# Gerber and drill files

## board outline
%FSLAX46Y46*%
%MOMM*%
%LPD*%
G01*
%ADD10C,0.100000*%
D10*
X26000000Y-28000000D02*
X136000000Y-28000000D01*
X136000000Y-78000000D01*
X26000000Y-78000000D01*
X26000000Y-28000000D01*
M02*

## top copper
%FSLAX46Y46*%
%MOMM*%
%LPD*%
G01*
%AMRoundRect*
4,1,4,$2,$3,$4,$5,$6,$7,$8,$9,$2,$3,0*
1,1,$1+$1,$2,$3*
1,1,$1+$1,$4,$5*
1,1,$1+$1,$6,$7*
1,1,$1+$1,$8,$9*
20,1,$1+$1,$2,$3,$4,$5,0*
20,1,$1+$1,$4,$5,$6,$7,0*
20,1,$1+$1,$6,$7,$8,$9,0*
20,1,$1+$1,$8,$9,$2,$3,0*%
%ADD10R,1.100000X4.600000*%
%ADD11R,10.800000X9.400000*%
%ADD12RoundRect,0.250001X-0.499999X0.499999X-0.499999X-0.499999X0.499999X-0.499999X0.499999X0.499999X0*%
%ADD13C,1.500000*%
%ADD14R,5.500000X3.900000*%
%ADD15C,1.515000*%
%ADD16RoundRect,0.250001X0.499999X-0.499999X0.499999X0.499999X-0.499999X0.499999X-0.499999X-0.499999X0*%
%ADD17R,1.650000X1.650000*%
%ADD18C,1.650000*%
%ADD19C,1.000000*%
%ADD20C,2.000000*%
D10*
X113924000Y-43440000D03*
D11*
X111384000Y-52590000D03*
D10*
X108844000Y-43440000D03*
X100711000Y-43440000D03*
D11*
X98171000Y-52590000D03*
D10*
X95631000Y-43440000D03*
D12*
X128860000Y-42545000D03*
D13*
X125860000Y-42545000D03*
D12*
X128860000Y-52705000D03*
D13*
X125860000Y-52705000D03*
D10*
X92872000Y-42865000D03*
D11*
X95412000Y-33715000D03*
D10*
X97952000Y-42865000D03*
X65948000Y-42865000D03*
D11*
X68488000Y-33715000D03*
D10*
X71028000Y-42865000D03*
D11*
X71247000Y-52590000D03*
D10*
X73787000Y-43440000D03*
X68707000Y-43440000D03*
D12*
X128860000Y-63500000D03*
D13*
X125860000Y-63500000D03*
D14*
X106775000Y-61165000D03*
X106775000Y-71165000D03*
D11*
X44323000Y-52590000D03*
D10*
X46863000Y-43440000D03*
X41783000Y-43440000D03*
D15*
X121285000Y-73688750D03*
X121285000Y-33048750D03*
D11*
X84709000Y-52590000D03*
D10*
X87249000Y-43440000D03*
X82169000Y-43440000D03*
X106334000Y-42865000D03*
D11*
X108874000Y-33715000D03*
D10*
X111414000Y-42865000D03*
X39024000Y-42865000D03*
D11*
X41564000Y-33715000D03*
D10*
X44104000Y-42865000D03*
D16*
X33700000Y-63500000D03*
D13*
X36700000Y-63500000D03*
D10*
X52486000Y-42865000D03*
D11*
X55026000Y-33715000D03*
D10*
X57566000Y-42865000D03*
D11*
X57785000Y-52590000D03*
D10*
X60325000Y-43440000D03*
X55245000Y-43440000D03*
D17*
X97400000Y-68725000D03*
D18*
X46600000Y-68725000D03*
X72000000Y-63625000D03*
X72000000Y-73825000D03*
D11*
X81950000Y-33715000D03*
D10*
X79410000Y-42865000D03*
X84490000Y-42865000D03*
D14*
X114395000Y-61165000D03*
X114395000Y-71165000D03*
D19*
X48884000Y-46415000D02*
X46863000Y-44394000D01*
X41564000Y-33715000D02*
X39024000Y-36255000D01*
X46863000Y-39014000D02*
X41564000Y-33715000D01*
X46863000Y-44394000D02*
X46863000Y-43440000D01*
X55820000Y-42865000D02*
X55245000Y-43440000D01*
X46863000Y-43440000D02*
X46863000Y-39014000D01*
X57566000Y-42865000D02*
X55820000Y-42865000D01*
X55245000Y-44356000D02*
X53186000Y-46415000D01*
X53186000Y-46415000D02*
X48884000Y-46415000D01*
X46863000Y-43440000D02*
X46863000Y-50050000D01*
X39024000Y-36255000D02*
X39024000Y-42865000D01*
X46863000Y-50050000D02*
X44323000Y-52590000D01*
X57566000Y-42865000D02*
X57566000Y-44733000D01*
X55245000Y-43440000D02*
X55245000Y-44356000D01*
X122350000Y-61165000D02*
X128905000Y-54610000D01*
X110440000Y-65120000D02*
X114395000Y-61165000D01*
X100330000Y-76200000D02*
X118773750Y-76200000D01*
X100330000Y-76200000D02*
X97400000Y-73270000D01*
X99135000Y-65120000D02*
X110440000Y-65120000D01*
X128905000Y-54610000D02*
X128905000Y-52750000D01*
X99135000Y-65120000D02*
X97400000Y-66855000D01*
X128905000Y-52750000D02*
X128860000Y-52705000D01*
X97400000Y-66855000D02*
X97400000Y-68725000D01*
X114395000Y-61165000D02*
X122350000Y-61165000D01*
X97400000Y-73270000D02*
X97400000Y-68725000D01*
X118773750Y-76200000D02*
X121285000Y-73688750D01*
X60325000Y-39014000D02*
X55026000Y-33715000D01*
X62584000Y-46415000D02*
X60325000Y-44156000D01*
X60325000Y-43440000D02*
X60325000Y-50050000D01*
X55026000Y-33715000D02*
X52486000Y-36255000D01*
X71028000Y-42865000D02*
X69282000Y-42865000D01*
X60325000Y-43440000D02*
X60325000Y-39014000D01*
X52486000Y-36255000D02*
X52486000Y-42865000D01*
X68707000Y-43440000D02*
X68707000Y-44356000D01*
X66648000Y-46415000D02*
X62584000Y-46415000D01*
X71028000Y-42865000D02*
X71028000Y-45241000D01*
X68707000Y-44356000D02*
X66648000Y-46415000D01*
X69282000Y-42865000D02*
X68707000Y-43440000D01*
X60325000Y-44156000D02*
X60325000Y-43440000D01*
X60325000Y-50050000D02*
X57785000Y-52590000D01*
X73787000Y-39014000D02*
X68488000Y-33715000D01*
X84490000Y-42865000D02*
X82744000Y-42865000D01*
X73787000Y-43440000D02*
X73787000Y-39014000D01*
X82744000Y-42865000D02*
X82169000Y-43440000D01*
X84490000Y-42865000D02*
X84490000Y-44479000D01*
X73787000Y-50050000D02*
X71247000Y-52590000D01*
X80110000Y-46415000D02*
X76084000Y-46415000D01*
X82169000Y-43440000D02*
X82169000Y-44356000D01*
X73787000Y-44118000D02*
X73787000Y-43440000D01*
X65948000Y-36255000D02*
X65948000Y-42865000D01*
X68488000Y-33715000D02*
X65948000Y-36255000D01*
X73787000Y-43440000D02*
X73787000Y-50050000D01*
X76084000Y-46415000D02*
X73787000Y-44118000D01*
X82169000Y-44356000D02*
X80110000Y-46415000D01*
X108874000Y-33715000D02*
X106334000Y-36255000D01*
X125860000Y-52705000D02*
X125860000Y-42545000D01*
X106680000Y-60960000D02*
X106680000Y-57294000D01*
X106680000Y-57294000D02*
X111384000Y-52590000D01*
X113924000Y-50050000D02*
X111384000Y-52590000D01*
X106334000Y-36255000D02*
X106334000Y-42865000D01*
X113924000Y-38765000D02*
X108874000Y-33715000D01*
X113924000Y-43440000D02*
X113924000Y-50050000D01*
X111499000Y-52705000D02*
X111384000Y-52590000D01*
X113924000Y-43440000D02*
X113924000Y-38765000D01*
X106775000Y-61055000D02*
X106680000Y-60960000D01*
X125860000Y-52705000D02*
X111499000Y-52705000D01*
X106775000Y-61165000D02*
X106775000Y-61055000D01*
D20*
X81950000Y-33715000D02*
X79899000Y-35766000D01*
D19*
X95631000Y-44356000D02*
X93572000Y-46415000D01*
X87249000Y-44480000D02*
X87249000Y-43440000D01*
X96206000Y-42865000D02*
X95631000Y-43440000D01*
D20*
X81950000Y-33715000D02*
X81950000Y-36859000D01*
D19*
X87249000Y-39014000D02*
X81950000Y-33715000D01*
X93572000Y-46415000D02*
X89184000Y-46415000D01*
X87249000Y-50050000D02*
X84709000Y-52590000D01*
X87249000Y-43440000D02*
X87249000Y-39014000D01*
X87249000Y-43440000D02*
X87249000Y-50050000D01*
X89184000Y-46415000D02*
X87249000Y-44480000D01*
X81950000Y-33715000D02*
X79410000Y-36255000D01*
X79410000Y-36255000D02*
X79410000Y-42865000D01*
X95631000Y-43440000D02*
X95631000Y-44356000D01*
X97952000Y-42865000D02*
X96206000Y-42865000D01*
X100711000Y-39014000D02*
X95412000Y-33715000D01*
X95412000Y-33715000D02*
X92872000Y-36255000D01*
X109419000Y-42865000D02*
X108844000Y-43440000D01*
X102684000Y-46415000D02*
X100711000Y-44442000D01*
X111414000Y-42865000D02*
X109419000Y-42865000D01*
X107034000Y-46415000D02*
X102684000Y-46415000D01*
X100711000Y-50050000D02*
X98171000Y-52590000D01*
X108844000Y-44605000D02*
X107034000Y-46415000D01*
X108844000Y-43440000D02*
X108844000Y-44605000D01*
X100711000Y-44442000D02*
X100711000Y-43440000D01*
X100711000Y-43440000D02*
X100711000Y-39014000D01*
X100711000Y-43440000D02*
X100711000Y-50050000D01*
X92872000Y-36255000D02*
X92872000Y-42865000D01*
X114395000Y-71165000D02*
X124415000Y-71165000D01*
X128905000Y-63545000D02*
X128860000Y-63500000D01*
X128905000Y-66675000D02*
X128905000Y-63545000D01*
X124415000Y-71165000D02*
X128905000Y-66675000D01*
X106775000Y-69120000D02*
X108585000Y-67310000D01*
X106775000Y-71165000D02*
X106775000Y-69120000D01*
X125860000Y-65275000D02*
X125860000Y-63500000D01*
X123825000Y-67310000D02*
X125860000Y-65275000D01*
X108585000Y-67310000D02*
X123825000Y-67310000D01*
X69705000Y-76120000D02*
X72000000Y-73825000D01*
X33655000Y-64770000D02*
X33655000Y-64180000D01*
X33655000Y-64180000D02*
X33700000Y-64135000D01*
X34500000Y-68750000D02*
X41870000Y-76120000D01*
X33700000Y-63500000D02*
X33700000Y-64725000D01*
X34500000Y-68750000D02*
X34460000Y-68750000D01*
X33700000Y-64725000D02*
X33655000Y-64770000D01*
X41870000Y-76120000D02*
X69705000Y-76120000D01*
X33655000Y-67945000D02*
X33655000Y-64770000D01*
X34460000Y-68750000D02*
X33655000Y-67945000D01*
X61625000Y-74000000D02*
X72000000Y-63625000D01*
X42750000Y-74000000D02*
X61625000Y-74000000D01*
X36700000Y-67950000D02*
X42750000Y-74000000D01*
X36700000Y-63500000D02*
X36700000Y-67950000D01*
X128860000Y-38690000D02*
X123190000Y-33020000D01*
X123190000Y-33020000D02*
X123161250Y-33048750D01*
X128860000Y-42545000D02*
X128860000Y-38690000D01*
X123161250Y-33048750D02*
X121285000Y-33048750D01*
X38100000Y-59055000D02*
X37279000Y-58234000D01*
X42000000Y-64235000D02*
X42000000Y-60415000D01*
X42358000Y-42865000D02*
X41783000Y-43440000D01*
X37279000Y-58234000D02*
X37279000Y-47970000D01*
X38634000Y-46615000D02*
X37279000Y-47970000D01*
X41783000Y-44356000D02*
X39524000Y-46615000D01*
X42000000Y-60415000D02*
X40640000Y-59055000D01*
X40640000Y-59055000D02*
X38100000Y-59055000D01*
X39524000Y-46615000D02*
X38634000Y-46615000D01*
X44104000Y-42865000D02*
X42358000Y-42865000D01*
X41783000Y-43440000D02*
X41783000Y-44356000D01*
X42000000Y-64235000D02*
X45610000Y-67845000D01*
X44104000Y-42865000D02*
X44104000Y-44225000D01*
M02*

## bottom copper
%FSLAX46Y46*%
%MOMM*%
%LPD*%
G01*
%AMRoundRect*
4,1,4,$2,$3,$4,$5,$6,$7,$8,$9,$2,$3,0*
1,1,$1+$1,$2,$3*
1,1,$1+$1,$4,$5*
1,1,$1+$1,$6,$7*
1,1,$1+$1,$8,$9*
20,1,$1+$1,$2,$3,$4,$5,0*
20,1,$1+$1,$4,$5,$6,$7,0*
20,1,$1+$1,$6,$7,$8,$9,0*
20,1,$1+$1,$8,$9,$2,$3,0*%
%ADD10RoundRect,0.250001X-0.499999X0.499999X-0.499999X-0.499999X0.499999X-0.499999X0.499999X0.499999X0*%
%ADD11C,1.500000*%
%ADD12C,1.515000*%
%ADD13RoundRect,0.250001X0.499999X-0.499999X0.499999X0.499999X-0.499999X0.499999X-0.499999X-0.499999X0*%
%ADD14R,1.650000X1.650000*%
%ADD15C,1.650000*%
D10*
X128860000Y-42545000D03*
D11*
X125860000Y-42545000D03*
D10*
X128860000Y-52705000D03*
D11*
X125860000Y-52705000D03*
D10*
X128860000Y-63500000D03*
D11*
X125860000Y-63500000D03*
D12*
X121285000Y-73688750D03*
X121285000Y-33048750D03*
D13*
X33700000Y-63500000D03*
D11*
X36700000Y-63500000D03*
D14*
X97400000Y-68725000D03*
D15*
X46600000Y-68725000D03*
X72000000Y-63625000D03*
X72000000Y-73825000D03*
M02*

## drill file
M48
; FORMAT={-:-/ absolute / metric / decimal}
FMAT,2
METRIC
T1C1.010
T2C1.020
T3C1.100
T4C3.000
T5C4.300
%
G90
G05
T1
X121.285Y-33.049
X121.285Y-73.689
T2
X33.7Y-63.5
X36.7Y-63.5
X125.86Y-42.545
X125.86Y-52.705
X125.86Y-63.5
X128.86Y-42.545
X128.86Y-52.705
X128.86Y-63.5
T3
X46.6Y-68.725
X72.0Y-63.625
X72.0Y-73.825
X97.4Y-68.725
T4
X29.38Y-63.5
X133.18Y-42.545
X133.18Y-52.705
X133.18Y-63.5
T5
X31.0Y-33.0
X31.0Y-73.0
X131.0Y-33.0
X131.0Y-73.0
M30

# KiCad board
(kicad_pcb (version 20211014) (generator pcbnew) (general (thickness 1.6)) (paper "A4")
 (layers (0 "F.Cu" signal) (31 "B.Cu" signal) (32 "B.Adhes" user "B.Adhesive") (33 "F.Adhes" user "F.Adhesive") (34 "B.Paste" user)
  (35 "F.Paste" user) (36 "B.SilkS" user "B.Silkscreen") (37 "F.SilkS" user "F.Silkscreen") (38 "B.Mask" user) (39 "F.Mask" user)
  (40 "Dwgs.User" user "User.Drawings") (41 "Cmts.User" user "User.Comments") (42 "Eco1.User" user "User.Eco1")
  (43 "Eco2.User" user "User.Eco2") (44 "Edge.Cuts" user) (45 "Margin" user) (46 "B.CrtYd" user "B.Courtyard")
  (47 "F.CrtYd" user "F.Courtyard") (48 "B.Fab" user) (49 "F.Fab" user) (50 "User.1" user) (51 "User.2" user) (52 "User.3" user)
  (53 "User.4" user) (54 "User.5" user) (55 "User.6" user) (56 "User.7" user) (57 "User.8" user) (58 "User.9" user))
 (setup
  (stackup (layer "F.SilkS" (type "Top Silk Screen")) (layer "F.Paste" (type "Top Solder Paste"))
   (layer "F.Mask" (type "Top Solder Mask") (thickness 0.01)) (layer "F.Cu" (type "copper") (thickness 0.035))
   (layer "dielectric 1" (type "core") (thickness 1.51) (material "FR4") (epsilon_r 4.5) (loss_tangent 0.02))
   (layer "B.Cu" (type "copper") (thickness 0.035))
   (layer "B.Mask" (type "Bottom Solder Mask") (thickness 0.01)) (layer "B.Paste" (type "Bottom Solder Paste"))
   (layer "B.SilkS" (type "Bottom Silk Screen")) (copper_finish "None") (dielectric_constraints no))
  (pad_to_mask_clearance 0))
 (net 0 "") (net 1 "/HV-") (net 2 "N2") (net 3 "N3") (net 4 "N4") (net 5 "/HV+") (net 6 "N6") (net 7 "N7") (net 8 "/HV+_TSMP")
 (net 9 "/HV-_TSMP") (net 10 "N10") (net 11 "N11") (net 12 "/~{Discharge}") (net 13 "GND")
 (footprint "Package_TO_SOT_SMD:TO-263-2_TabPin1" (layer "F.Cu") (at 111.384 49.215 -90)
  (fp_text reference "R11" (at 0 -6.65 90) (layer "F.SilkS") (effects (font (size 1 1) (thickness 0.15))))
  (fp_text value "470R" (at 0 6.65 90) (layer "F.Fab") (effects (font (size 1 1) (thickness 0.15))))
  (pad "" smd rect (at 5.8 2.775 270) (size 4.55 5.25) (layers "F.Paste"))
  (pad "" smd rect (at 5.8 -2.775 270) (size 4.55 5.25) (layers "F.Paste"))
  (pad "" smd rect (at 0.95 -2.775 270) (size 4.55 5.25) (layers "F.Paste"))
  (pad "" smd rect (at 0.95 2.775 270) (size 4.55 5.25) (layers "F.Paste"))
  (pad "1" smd rect (at -5.775 -2.54 270) (size 4.6 1.1) (layers "F.Cu" "F.Paste" "F.Mask") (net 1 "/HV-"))
  (pad "1" smd rect (at 3.375 0 270) (size 9.4 10.8) (layers "F.Cu" "F.Mask") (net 1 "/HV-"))
  (pad "2" smd rect (at -5.775 2.54 270) (size 4.6 1.1) (layers "F.Cu" "F.Paste" "F.Mask") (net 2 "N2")))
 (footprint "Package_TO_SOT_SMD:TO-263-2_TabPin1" (layer "F.Cu") (at 98.171 49.215 -90)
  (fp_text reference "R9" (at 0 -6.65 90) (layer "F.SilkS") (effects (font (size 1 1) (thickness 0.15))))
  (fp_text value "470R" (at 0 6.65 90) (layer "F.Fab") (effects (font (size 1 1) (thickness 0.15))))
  (pad "" smd rect (at 0.95 -2.775 270) (size 4.55 5.25) (layers "F.Paste"))
  (pad "" smd rect (at 5.8 2.775 270) (size 4.55 5.25) (layers "F.Paste"))
  (pad "" smd rect (at 0.95 2.775 270) (size 4.55 5.25) (layers "F.Paste"))
  (pad "" smd rect (at 5.8 -2.775 270) (size 4.55 5.25) (layers "F.Paste"))
  (pad "1" smd rect (at -5.775 -2.54 270) (size 4.6 1.1) (layers "F.Cu" "F.Paste" "F.Mask") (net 2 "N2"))
  (pad "1" smd rect (at 3.375 0 270) (size 9.4 10.8) (layers "F.Cu" "F.Mask") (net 2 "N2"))
  (pad "2" smd rect (at -5.775 2.54 270) (size 4.6 1.1) (layers "F.Cu" "F.Paste" "F.Mask") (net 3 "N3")))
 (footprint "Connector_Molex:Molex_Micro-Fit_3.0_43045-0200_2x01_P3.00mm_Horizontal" (layer "F.Cu") (at 128.86 42.545 -90)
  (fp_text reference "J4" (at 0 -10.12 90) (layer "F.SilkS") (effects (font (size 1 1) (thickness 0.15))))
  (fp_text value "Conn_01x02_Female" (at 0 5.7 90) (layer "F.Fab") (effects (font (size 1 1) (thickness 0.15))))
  (pad "" np_thru_hole circle (at 0 -4.32 270) (size 3 3) (drill 3) (layers *.Cu *.Mask))
  (pad "1" thru_hole roundrect (at 0 0 270) (size 1.5 1.5) (drill 1.02) (layers *.Cu *.Mask) (roundrect_rratio 0.166667) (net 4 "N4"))
  (pad "2" thru_hole circle (at 0 3 270) (size 1.5 1.5) (drill 1.02) (layers *.Cu *.Mask) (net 1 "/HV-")))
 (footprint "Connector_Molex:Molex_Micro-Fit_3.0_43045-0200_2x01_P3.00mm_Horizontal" (layer "F.Cu") (at 128.86 52.705 -90)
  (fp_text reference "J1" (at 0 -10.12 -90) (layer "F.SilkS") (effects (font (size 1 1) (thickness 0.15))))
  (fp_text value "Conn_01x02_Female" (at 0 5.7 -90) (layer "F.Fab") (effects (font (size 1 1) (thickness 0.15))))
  (pad "" np_thru_hole circle (at 0 -4.32 270) (size 3 3) (drill 3) (layers *.Cu *.Mask))
  (pad "1" thru_hole roundrect (at 0 0 270) (size 1.5 1.5) (drill 1.02) (layers *.Cu *.Mask) (roundrect_rratio 0.1666673333) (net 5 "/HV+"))
  (pad "2" thru_hole circle (at 0 3 270) (size 1.5 1.5) (drill 1.02) (layers *.Cu *.Mask) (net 1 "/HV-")))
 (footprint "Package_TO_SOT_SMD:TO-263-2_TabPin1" (layer "F.Cu") (at 95.412 37.09 90)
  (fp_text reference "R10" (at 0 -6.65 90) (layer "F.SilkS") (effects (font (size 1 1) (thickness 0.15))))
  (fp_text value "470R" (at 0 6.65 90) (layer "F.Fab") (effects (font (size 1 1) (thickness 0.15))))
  (pad "" smd rect (at 5.8 -2.775 90) (size 4.55 5.25) (layers "F.Paste"))
  (pad "" smd rect (at 0.95 2.775 90) (size 4.55 5.25) (layers "F.Paste"))
  (pad "" smd rect (at 0.95 -2.775 90) (size 4.55 5.25) (layers "F.Paste"))
  (pad "" smd rect (at 5.8 2.775 90) (size 4.55 5.25) (layers "F.Paste"))
  (pad "1" smd rect (at -5.775 -2.54 90) (size 4.6 1.1) (layers "F.Cu" "F.Paste" "F.Mask") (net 2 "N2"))
  (pad "1" smd rect (at 3.375 0 90) (size 9.4 10.8) (layers "F.Cu" "F.Mask") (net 2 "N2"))
  (pad "2" smd rect (at -5.775 2.54 90) (size 4.6 1.1) (layers "F.Cu" "F.Paste" "F.Mask") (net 3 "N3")))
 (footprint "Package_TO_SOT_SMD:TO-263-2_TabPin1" (layer "F.Cu") (at 68.488 37.09 90)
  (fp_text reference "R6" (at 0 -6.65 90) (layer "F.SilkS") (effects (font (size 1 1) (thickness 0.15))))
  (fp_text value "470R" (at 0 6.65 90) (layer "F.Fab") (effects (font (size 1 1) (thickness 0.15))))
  (pad "" smd rect (at 0.95 2.775 90) (size 4.55 5.25) (layers "F.Paste"))
  (pad "" smd rect (at 5.8 -2.775 90) (size 4.55 5.25) (layers "F.Paste"))
  (pad "" smd rect (at 0.95 -2.775 90) (size 4.55 5.25) (layers "F.Paste"))
  (pad "" smd rect (at 5.8 2.775 90) (size 4.55 5.25) (layers "F.Paste"))
  (pad "1" smd rect (at -5.775 -2.54 90) (size 4.6 1.1) (layers "F.Cu" "F.Paste" "F.Mask") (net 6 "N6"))
  (pad "1" smd rect (at 3.375 0 90) (size 9.4 10.8) (layers "F.Cu" "F.Mask") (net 6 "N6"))
  (pad "2" smd rect (at -5.775 2.54 90) (size 4.6 1.1) (layers "F.Cu" "F.Paste" "F.Mask") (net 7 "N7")))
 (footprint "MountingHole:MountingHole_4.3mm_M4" (layer "F.Cu") (at 131 73)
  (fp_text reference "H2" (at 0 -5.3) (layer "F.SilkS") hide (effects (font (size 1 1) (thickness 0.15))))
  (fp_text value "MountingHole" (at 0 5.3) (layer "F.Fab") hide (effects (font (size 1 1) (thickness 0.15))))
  (pad "" np_thru_hole circle (at 0 0) (size 4.3 4.3) (drill 4.3) (layers *.Cu *.Mask)))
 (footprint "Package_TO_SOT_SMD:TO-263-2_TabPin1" (layer "F.Cu") (at 71.247 49.215 -90)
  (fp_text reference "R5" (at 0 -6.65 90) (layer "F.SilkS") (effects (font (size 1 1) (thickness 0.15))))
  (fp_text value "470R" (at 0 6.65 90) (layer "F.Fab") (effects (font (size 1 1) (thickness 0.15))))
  (pad "" smd rect (at 0.95 2.775 270) (size 4.55 5.25) (layers "F.Paste"))
  (pad "" smd rect (at 5.8 2.775 270) (size 4.55 5.25) (layers "F.Paste"))
  (pad "" smd rect (at 0.95 -2.775 270) (size 4.55 5.25) (layers "F.Paste"))
  (pad "" smd rect (at 5.8 -2.775 270) (size 4.55 5.25) (layers "F.Paste"))
  (pad "1" smd rect (at 3.375 0 270) (size 9.4 10.8) (layers "F.Cu" "F.Mask") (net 6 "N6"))
  (pad "1" smd rect (at -5.775 -2.54 270) (size 4.6 1.1) (layers "F.Cu" "F.Paste" "F.Mask") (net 6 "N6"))
  (pad "2" smd rect (at -5.775 2.54 270) (size 4.6 1.1) (layers "F.Cu" "F.Paste" "F.Mask") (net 7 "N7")))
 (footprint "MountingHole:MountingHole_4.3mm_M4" (layer "F.Cu") (at 31 73)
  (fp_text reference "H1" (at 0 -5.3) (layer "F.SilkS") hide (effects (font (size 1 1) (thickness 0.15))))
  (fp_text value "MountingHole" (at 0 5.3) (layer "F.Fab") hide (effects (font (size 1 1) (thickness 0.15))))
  (pad "" np_thru_hole circle (at 0 0) (size 4.3 4.3) (drill 4.3) (layers *.Cu *.Mask)))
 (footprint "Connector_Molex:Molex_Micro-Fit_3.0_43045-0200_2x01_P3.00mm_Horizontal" (layer "F.Cu") (at 128.86 63.5 -90)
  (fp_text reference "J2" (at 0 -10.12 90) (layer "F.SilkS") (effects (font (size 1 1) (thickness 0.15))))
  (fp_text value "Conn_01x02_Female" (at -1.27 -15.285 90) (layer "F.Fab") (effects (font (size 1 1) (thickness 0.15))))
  (pad "" np_thru_hole circle (at 0 -4.32 270) (size 3 3) (drill 3) (layers *.Cu *.Mask))
  (pad "1" thru_hole roundrect (at 0 0 270) (size 1.5 1.5) (drill 1.02) (layers *.Cu *.Mask) (roundrect_rratio 0.1666673333)
   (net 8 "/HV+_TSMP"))
  (pad "2" thru_hole circle (at 0 3 270) (size 1.5 1.5) (drill 1.02) (layers *.Cu *.Mask) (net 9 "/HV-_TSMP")))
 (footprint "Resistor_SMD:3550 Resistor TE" (layer "F.Cu") (at 104.025 59.215 -90)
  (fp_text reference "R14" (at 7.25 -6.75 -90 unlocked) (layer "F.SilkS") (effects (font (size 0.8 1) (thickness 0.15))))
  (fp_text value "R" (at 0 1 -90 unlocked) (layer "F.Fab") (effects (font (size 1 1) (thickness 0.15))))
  (pad "1" smd rect (at 1.95 -2.75 270) (size 3.9 5.5) (layers "F.Cu" "F.Paste" "F.Mask") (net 1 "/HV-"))
  (pad "2" smd rect (at 11.95 -2.75 270) (size 3.9 5.5) (layers "F.Cu" "F.Paste" "F.Mask") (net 9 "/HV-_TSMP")))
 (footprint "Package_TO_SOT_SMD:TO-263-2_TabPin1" (layer "F.Cu") (at 44.323 49.215 -90)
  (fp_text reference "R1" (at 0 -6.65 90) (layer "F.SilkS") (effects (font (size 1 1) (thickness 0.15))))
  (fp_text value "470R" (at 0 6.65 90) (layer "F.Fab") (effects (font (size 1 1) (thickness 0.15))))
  (pad "" smd rect (at 0.95 -2.775 270) (size 4.55 5.25) (layers "F.Paste"))
  (pad "" smd rect (at 5.8 2.775 270) (size 4.55 5.25) (layers "F.Paste"))
  (pad "" smd rect (at 5.8 -2.775 270) (size 4.55 5.25) (layers "F.Paste"))
  (pad "" smd rect (at 0.95 2.775 270) (size 4.55 5.25) (layers "F.Paste"))
  (pad "1" smd rect (at 3.375 0 270) (size 9.4 10.8) (layers "F.Cu" "F.Mask") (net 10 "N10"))
  (pad "1" smd rect (at -5.775 -2.54 270) (size 4.6 1.1) (layers "F.Cu" "F.Paste" "F.Mask") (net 10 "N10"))
  (pad "2" smd rect (at -5.775 2.54 270) (size 4.6 1.1) (layers "F.Cu" "F.Paste" "F.Mask") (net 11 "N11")))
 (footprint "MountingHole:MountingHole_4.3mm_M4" (layer "F.Cu") (at 131 33)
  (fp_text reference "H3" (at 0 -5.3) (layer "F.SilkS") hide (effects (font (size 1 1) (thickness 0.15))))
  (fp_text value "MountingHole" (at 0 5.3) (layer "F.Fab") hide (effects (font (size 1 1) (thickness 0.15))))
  (pad "" np_thru_hole circle (at 0 0) (size 4.3 4.3) (drill 4.3) (layers *.Cu *.Mask)))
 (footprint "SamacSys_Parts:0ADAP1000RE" (layer "F.Cu") (at 121.285 75.40875 90)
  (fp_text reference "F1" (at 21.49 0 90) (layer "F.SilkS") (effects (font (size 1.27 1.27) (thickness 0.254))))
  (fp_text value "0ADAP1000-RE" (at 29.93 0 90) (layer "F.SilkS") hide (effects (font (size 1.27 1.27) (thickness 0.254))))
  (pad "1" thru_hole circle (at 1.72 0 90) (size 1.515 1.515) (drill 1.01) (layers *.Cu *.Mask) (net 5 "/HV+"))
  (pad "2" thru_hole circle (at 42.36 0 90) (size 1.515 1.515) (drill 1.01) (layers *.Cu *.Mask) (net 4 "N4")))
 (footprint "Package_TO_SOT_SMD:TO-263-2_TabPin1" (layer "F.Cu") (at 84.709 49.215 -90)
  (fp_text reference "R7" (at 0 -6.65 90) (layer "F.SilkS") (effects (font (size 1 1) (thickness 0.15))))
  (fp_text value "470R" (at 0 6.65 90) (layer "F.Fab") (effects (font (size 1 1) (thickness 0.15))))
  (pad "" smd rect (at 0.95 2.775 270) (size 4.55 5.25) (layers "F.Paste"))
  (pad "" smd rect (at 0.95 -2.775 270) (size 4.55 5.25) (layers "F.Paste"))
  (pad "" smd rect (at 5.8 2.775 270) (size 4.55 5.25) (layers "F.Paste"))
  (pad "" smd rect (at 5.8 -2.775 270) (size 4.55 5.25) (layers "F.Paste"))
  (pad "1" smd rect (at 3.375 0 270) (size 9.4 10.8) (layers "F.Cu" "F.Mask") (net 3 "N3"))
  (pad "1" smd rect (at -5.775 -2.54 270) (size 4.6 1.1) (layers "F.Cu" "F.Paste" "F.Mask") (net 3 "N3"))
  (pad "2" smd rect (at -5.775 2.54 270) (size 4.6 1.1) (layers "F.Cu" "F.Paste" "F.Mask") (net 6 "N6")))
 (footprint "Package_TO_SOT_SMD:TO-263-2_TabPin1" (layer "F.Cu") (at 108.874 37.09 90)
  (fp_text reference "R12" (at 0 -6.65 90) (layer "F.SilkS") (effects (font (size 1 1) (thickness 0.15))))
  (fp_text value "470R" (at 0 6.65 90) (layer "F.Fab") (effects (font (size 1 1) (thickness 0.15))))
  (pad "" smd rect (at 5.8 2.775 90) (size 4.55 5.25) (layers "F.Paste"))
  (pad "" smd rect (at 0.95 -2.775 90) (size 4.55 5.25) (layers "F.Paste"))
  (pad "" smd rect (at 5.8 -2.775 90) (size 4.55 5.25) (layers "F.Paste"))
  (pad "" smd rect (at 0.95 2.775 90) (size 4.55 5.25) (layers "F.Paste"))
  (pad "1" smd rect (at -5.775 -2.54 90) (size 4.6 1.1) (layers "F.Cu" "F.Paste" "F.Mask") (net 1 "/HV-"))
  (pad "1" smd rect (at 3.375 0 90) (size 9.4 10.8) (layers "F.Cu" "F.Mask") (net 1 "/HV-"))
  (pad "2" smd rect (at -5.775 2.54 90) (size 4.6 1.1) (layers "F.Cu" "F.Paste" "F.Mask") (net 2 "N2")))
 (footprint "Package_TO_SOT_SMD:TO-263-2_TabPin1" (layer "F.Cu") (at 41.564 37.09 90)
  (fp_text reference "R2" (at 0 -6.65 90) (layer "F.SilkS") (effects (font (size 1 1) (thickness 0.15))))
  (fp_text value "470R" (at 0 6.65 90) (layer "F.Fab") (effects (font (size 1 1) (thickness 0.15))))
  (pad "" smd rect (at 5.8 2.775 90) (size 4.55 5.25) (layers "F.Paste"))
  (pad "" smd rect (at 5.8 -2.775 90) (size 4.55 5.25) (layers "F.Paste"))
  (pad "" smd rect (at 0.95 2.775 90) (size 4.55 5.25) (layers "F.Paste"))
  (pad "" smd rect (at 0.95 -2.775 90) (size 4.55 5.25) (layers "F.Paste"))
  (pad "1" smd rect (at -5.775 -2.54 90) (size 4.6 1.1) (layers "F.Cu" "F.Paste" "F.Mask") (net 10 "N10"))
  (pad "1" smd rect (at 3.375 0 90) (size 9.4 10.8) (layers "F.Cu" "F.Mask") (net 10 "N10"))
  (pad "2" smd rect (at -5.775 2.54 90) (size 4.6 1.1) (layers "F.Cu" "F.Paste" "F.Mask") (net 11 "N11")))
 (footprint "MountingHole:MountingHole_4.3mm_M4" (layer "F.Cu") (at 31 33)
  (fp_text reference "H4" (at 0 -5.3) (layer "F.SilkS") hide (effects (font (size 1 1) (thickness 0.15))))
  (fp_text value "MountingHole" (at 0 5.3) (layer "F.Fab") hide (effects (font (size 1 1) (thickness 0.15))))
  (pad "" np_thru_hole circle (at 0 0) (size 4.3 4.3) (drill 4.3) (layers *.Cu *.Mask)))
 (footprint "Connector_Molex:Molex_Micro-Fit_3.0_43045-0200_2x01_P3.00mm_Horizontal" (layer "F.Cu") (at 33.7 63.5 90)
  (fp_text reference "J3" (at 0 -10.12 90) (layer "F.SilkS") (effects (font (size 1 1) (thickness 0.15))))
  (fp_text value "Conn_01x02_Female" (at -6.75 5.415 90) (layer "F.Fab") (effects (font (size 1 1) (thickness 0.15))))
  (pad "" np_thru_hole circle (at 0 -4.32 90) (size 3 3) (drill 3) (layers *.Cu *.Mask))
  (pad "1" thru_hole roundrect (at 0 0 90) (size 1.5 1.5) (drill 1.02) (layers *.Cu *.Mask) (roundrect_rratio 0.1666673333)
   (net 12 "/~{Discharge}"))
  (pad "2" thru_hole circle (at 0 3 90) (size 1.5 1.5) (drill 1.02) (layers *.Cu *.Mask) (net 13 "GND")))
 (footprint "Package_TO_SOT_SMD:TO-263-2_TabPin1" (layer "F.Cu") (at 55.026 37.09 90)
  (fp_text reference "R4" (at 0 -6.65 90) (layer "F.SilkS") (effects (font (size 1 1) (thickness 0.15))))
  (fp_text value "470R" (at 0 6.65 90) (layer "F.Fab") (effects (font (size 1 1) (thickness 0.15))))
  (pad "" smd rect (at 0.95 -2.775 90) (size 4.55 5.25) (layers "F.Paste"))
  (pad "" smd rect (at 0.95 2.775 90) (size 4.55 5.25) (layers "F.Paste"))
  (pad "" smd rect (at 5.8 -2.775 90) (size 4.55 5.25) (layers "F.Paste"))
  (pad "" smd rect (at 5.8 2.775 90) (size 4.55 5.25) (layers "F.Paste"))
  (pad "1" smd rect (at -5.775 -2.54 90) (size 4.6 1.1) (layers "F.Cu" "F.Paste" "F.Mask") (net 7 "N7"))
  (pad "1" smd rect (at 3.375 0 90) (size 9.4 10.8) (layers "F.Cu" "F.Mask") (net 7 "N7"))
  (pad "2" smd rect (at -5.775 2.54 90) (size 4.6 1.1) (layers "F.Cu" "F.Paste" "F.Mask") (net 10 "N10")))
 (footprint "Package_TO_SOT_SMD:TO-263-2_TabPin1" (layer "F.Cu") (at 57.785 49.215 -90)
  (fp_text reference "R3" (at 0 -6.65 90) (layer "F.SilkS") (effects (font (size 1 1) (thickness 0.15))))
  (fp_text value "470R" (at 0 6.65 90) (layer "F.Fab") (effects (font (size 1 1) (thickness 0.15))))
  (pad "" smd rect (at 5.8 -2.775 270) (size 4.55 5.25) (layers "F.Paste"))
  (pad "" smd rect (at 0.95 2.775 270) (size 4.55 5.25) (layers "F.Paste"))
  (pad "" smd rect (at 5.8 2.775 270) (size 4.55 5.25) (layers "F.Paste"))
  (pad "" smd rect (at 0.95 -2.775 270) (size 4.55 5.25) (layers "F.Paste"))
  (pad "1" smd rect (at 3.375 0 270) (size 9.4 10.8) (layers "F.Cu" "F.Mask") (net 7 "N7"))
  (pad "1" smd rect (at -5.775 -2.54 270) (size 4.6 1.1) (layers "F.Cu" "F.Paste" "F.Mask") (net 7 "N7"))
  (pad "2" smd rect (at -5.775 2.54 270) (size 4.6 1.1) (layers "F.Cu" "F.Paste" "F.Mask") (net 10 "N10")))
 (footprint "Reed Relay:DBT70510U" (layer "F.Cu") (at 97.4 68.725 180)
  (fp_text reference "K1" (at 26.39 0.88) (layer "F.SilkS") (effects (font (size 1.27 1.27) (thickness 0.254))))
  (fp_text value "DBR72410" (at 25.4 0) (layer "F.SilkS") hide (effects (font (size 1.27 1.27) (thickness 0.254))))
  (pad "1" thru_hole rect locked (at 0 0 180) (size 1.65 1.65) (drill 1.1) (layers *.Cu *.Mask) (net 5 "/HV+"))
  (pad "2" thru_hole circle locked (at 50.8 0 180) (size 1.65 1.65) (drill 1.1) (layers *.Cu *.Mask) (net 11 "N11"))
  (pad "3" thru_hole circle locked (at 25.4 5.1 180) (size 1.65 1.65) (drill 1.1) (layers *.Cu *.Mask) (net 13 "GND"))
  (pad "4" thru_hole circle locked (at 25.4 -5.1 180) (size 1.65 1.65) (drill 1.1) (layers *.Cu *.Mask) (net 12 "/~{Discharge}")))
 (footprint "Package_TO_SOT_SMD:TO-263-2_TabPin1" (layer "F.Cu") (at 81.95 37.09 90)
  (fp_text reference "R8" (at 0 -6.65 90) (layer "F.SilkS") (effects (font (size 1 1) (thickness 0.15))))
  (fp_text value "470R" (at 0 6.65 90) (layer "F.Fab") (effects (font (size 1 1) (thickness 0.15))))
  (pad "" smd rect (at 0.95 2.775 90) (size 4.55 5.25) (layers "F.Paste"))
  (pad "" smd rect (at 5.8 2.775 90) (size 4.55 5.25) (layers "F.Paste"))
  (pad "" smd rect (at 0.95 -2.775 90) (size 4.55 5.25) (layers "F.Paste"))
  (pad "" smd rect (at 5.8 -2.775 90) (size 4.55 5.25) (layers "F.Paste"))
  (pad "1" smd rect (at 3.375 0 90) (size 9.4 10.8) (layers "F.Cu" "F.Mask") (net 3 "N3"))
  (pad "1" smd rect (at -5.775 -2.54 90) (size 4.6 1.1) (layers "F.Cu" "F.Paste" "F.Mask") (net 3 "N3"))
  (pad "2" smd rect (at -5.775 2.54 90) (size 4.6 1.1) (layers "F.Cu" "F.Paste" "F.Mask") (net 6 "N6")))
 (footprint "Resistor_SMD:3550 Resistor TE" (layer "F.Cu") (at 111.645 59.215 -90)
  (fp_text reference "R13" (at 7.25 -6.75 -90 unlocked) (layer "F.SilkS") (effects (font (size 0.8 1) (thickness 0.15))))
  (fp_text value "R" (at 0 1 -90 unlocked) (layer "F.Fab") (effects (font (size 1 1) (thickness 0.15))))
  (pad "1" smd rect (at 1.95 -2.75 270) (size 3.9 5.5) (layers "F.Cu" "F.Paste" "F.Mask") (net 5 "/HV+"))
  (pad "2" smd rect (at 11.95 -2.75 270) (size 3.9 5.5) (layers "F.Cu" "F.Paste" "F.Mask") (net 8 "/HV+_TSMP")))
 (gr_rect (start 26 28) (end 136 78) (layer "Edge.Cuts") (width 0.1) (fill none))
 (segment (start 48.884 46.415) (end 46.863 44.394) (width 1) (layer "F.Cu") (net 10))
 (segment (start 41.564 33.715) (end 39.024 36.255) (width 1) (layer "F.Cu") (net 10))
 (segment (start 46.863 39.014) (end 41.564 33.715) (width 1) (layer "F.Cu") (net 10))
 (segment (start 46.863 44.394) (end 46.863 43.44) (width 1) (layer "F.Cu") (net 10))
 (segment (start 55.82 42.865) (end 55.245 43.44) (width 1) (layer "F.Cu") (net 10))
 (segment (start 46.863 43.44) (end 46.863 39.014) (width 1) (layer "F.Cu") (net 10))
 (segment (start 57.566 42.865) (end 55.82 42.865) (width 1) (layer "F.Cu") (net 10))
 (segment (start 55.245 44.356) (end 53.186 46.415) (width 1) (layer "F.Cu") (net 10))
 (segment (start 53.186 46.415) (end 48.884 46.415) (width 1) (layer "F.Cu") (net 10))
 (segment (start 46.863 43.44) (end 46.863 50.05) (width 1) (layer "F.Cu") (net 10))
 (segment (start 39.024 36.255) (end 39.024 42.865) (width 1) (layer "F.Cu") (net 10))
 (segment (start 46.863 50.05) (end 44.323 52.59) (width 1) (layer "F.Cu") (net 10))
 (segment (start 57.566 42.865) (end 57.566 44.733) (width 1) (layer "F.Cu") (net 10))
 (segment (start 55.245 43.44) (end 55.245 44.356) (width 1) (layer "F.Cu") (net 10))
 (segment (start 122.35 61.165) (end 128.905 54.61) (width 1) (layer "F.Cu") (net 5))
 (segment (start 110.44 65.12) (end 114.395 61.165) (width 1) (layer "F.Cu") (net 5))
 (segment (start 100.33 76.2) (end 118.77375 76.2) (width 1) (layer "F.Cu") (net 5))
 (segment (start 100.33 76.2) (end 97.4 73.27) (width 1) (layer "F.Cu") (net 5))
 (segment (start 99.135 65.12) (end 110.44 65.12) (width 1) (layer "F.Cu") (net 5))
 (segment (start 128.905 54.61) (end 128.905 52.75) (width 1) (layer "F.Cu") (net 5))
 (segment (start 99.135 65.12) (end 97.4 66.855) (width 1) (layer "F.Cu") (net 5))
 (segment (start 128.905 52.75) (end 128.86 52.705) (width 1) (layer "F.Cu") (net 5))
 (segment (start 97.4 66.855) (end 97.4 68.725) (width 1) (layer "F.Cu") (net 5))
 (segment (start 114.395 61.165) (end 122.35 61.165) (width 1) (layer "F.Cu") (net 5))
 (segment (start 97.4 73.27) (end 97.4 68.725) (width 1) (layer "F.Cu") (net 5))
 (segment (start 118.77375 76.2) (end 121.285 73.68875) (width 1) (layer "F.Cu") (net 5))
 (segment (start 60.325 39.014) (end 55.026 33.715) (width 1) (layer "F.Cu") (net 7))
 (segment (start 62.584 46.415) (end 60.325 44.156) (width 1) (layer "F.Cu") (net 7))
 (segment (start 60.325 43.44) (end 60.325 50.05) (width 1) (layer "F.Cu") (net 7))
 (segment (start 55.026 33.715) (end 52.486 36.255) (width 1) (layer "F.Cu") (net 7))
 (segment (start 71.028 42.865) (end 69.282 42.865) (width 1) (layer "F.Cu") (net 7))
 (segment (start 60.325 43.44) (end 60.325 39.014) (width 1) (layer "F.Cu") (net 7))
 (segment (start 52.486 36.255) (end 52.486 42.865) (width 1) (layer "F.Cu") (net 7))
 (segment (start 68.707 43.44) (end 68.707 44.356) (width 1) (layer "F.Cu") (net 7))
 (segment (start 66.648 46.415) (end 62.584 46.415) (width 1) (layer "F.Cu") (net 7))
 (segment (start 71.028 42.865) (end 71.028 45.241) (width 1) (layer "F.Cu") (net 7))
 (segment (start 68.707 44.356) (end 66.648 46.415) (width 1) (layer "F.Cu") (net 7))
 (segment (start 69.282 42.865) (end 68.707 43.44) (width 1) (layer "F.Cu") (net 7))
 (segment (start 60.325 44.156) (end 60.325 43.44) (width 1) (layer "F.Cu") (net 7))
 (segment (start 60.325 50.05) (end 57.785 52.59) (width 1) (layer "F.Cu") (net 7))
 (segment (start 73.787 39.014) (end 68.488 33.715) (width 1) (layer "F.Cu") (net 6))
 (segment (start 84.49 42.865) (end 82.744 42.865) (width 1) (layer "F.Cu") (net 6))
 (segment (start 73.787 43.44) (end 73.787 39.014) (width 1) (layer "F.Cu") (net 6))
 (segment (start 82.744 42.865) (end 82.169 43.44) (width 1) (layer "F.Cu") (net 6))
 (segment (start 84.49 42.865) (end 84.49 44.479) (width 1) (layer "F.Cu") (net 6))
 (segment (start 73.787 50.05) (end 71.247 52.59) (width 1) (layer "F.Cu") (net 6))
 (segment (start 80.11 46.415) (end 76.084 46.415) (width 1) (layer "F.Cu") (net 6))
 (segment (start 82.169 43.44) (end 82.169 44.356) (width 1) (layer "F.Cu") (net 6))
 (segment (start 73.787 44.118) (end 73.787 43.44) (width 1) (layer "F.Cu") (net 6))
 (segment (start 65.948 36.255) (end 65.948 42.865) (width 1) (layer "F.Cu") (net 6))
 (segment (start 68.488 33.715) (end 65.948 36.255) (width 1) (layer "F.Cu") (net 6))
 (segment (start 73.787 43.44) (end 73.787 50.05) (width 1) (layer "F.Cu") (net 6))
 (segment (start 76.084 46.415) (end 73.787 44.118) (width 1) (layer "F.Cu") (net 6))
 (segment (start 82.169 44.356) (end 80.11 46.415) (width 1) (layer "F.Cu") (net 6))
 (segment (start 108.874 33.715) (end 106.334 36.255) (width 1) (layer "F.Cu") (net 1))
 (segment (start 125.86 52.705) (end 125.86 42.545) (width 1) (layer "F.Cu") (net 1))
 (segment (start 106.68 60.96) (end 106.68 57.294) (width 1) (layer "F.Cu") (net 1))
 (segment (start 106.68 57.294) (end 111.384 52.59) (width 1) (layer "F.Cu") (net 1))
 (segment (start 113.924 50.05) (end 111.384 52.59) (width 1) (layer "F.Cu") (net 1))
 (segment (start 106.334 36.255) (end 106.334 42.865) (width 1) (layer "F.Cu") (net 1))
 (segment (start 113.924 38.765) (end 108.874 33.715) (width 1) (layer "F.Cu") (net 1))
 (segment (start 113.924 43.44) (end 113.924 50.05) (width 1) (layer "F.Cu") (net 1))
 (segment (start 111.499 52.705) (end 111.384 52.59) (width 1) (layer "F.Cu") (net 1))
 (segment (start 113.924 43.44) (end 113.924 38.765) (width 1) (layer "F.Cu") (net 1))
 (segment (start 106.775 61.055) (end 106.68 60.96) (width 1) (layer "F.Cu") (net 1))
 (segment (start 125.86 52.705) (end 111.499 52.705) (width 1) (layer "F.Cu") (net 1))
 (segment (start 106.775 61.165) (end 106.775 61.055) (width 1) (layer "F.Cu") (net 1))
 (segment (start 81.95 33.715) (end 79.899 35.766) (width 2) (layer "F.Cu") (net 3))
 (segment (start 95.631 44.356) (end 93.572 46.415) (width 1) (layer "F.Cu") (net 3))
 (segment (start 87.249 44.48) (end 87.249 43.44) (width 1) (layer "F.Cu") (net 3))
 (segment (start 96.206 42.865) (end 95.631 43.44) (width 1) (layer "F.Cu") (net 3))
 (segment (start 81.95 33.715) (end 81.95 36.859) (width 2) (layer "F.Cu") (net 3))
 (segment (start 87.249 39.014) (end 81.95 33.715) (width 1) (layer "F.Cu") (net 3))
 (segment (start 93.572 46.415) (end 89.184 46.415) (width 1) (layer "F.Cu") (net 3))
 (segment (start 87.249 50.05) (end 84.709 52.59) (width 1) (layer "F.Cu") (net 3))
 (segment (start 87.249 43.44) (end 87.249 39.014) (width 1) (layer "F.Cu") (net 3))
 (segment (start 87.249 43.44) (end 87.249 50.05) (width 1) (layer "F.Cu") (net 3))
 (segment (start 89.184 46.415) (end 87.249 44.48) (width 1) (layer "F.Cu") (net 3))
 (segment (start 81.95 33.715) (end 79.41 36.255) (width 1) (layer "F.Cu") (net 3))
 (segment (start 79.41 36.255) (end 79.41 42.865) (width 1) (layer "F.Cu") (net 3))
 (segment (start 95.631 43.44) (end 95.631 44.356) (width 1) (layer "F.Cu") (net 3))
 (segment (start 97.952 42.865) (end 96.206 42.865) (width 1) (layer "F.Cu") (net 3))
 (segment (start 100.711 39.014) (end 95.412 33.715) (width 1) (layer "F.Cu") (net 2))
 (segment (start 95.412 33.715) (end 92.872 36.255) (width 1) (layer "F.Cu") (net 2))
 (segment (start 109.419 42.865) (end 108.844 43.44) (width 1) (layer "F.Cu") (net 2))
 (segment (start 102.684 46.415) (end 100.711 44.442) (width 1) (layer "F.Cu") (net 2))
 (segment (start 111.414 42.865) (end 109.419 42.865) (width 1) (layer "F.Cu") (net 2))
 (segment (start 107.034 46.415) (end 102.684 46.415) (width 1) (layer "F.Cu") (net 2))
 (segment (start 100.711 50.05) (end 98.171 52.59) (width 1) (layer "F.Cu") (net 2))
 (segment (start 108.844 44.605) (end 107.034 46.415) (width 1) (layer "F.Cu") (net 2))
 (segment (start 108.844 43.44) (end 108.844 44.605) (width 1) (layer "F.Cu") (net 2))
 (segment (start 100.711 44.442) (end 100.711 43.44) (width 1) (layer "F.Cu") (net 2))
 (segment (start 100.711 43.44) (end 100.711 39.014) (width 1) (layer "F.Cu") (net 2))
 (segment (start 100.711 43.44) (end 100.711 50.05) (width 1) (layer "F.Cu") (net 2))
 (segment (start 92.872 36.255) (end 92.872 42.865) (width 1) (layer "F.Cu") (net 2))
 (segment (start 114.395 71.165) (end 124.415 71.165) (width 1) (layer "F.Cu") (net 8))
 (segment (start 128.905 63.545) (end 128.86 63.5) (width 1) (layer "F.Cu") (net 8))
 (segment (start 128.905 66.675) (end 128.905 63.545) (width 1) (layer "F.Cu") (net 8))
 (segment (start 124.415 71.165) (end 128.905 66.675) (width 1) (layer "F.Cu") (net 8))
 (segment (start 106.775 69.12) (end 108.585 67.31) (width 1) (layer "F.Cu") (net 9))
 (segment (start 106.775 71.165) (end 106.775 69.12) (width 1) (layer "F.Cu") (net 9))
 (segment (start 125.86 65.275) (end 125.86 63.5) (width 1) (layer "F.Cu") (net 9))
 (segment (start 123.825 67.31) (end 125.86 65.275) (width 1) (layer "F.Cu") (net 9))
 (segment (start 108.585 67.31) (end 123.825 67.31) (width 1) (layer "F.Cu") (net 9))
 (segment (start 69.705 76.12) (end 72 73.825) (width 1) (layer "F.Cu") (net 12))
 (segment (start 33.655 64.77) (end 33.655 64.18) (width 1) (layer "F.Cu") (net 12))
 (segment (start 33.655 64.18) (end 33.7 64.135) (width 1) (layer "F.Cu") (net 12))
 (segment (start 34.5 68.75) (end 41.87 76.12) (width 1) (layer "F.Cu") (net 12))
 (segment (start 33.7 63.5) (end 33.7 64.725) (width 1) (layer "F.Cu") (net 12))
 (segment (start 34.5 68.75) (end 34.46 68.75) (width 1) (layer "F.Cu") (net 12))
 (segment (start 33.7 64.725) (end 33.655 64.77) (width 1) (layer "F.Cu") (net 12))
 (segment (start 41.87 76.12) (end 69.705 76.12) (width 1) (layer "F.Cu") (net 12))
 (segment (start 33.655 67.945) (end 33.655 64.77) (width 1) (layer "F.Cu") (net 12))
 (segment (start 34.46 68.75) (end 33.655 67.945) (width 1) (layer "F.Cu") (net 12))
 (segment (start 61.625 74) (end 72 63.625) (width 1) (layer "F.Cu") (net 13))
 (segment (start 42.75 74) (end 61.625 74) (width 1) (layer "F.Cu") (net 13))
 (segment (start 36.7 67.95) (end 42.75 74) (width 1) (layer "F.Cu") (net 13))
 (segment (start 36.7 63.5) (end 36.7 67.95) (width 1) (layer "F.Cu") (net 13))
 (segment (start 128.86 38.69) (end 123.19 33.02) (width 1) (layer "F.Cu") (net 4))
 (segment (start 123.19 33.02) (end 123.16125 33.04875) (width 1) (layer "F.Cu") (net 4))
 (segment (start 128.86 42.545) (end 128.86 38.69) (width 1) (layer "F.Cu") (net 4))
 (segment (start 123.16125 33.04875) (end 121.285 33.04875) (width 1) (layer "F.Cu") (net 4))
 (segment (start 38.1 59.055) (end 37.279 58.234) (width 1) (layer "F.Cu") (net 11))
 (segment (start 42 64.235) (end 42 60.415) (width 1) (layer "F.Cu") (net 11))
 (segment (start 42.358 42.865) (end 41.783 43.44) (width 1) (layer "F.Cu") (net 11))
 (segment (start 37.279 58.234) (end 37.279 47.97) (width 1) (layer "F.Cu") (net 11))
 (segment (start 38.634 46.615) (end 37.279 47.97) (width 1) (layer "F.Cu") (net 11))
 (segment (start 41.783 44.356) (end 39.524 46.615) (width 1) (layer "F.Cu") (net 11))
 (segment (start 42 60.415) (end 40.64 59.055) (width 1) (layer "F.Cu") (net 11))
 (segment (start 40.64 59.055) (end 38.1 59.055) (width 1) (layer "F.Cu") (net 11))
 (segment (start 39.524 46.615) (end 38.634 46.615) (width 1) (layer "F.Cu") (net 11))
 (segment (start 44.104 42.865) (end 42.358 42.865) (width 1) (layer "F.Cu") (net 11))
 (segment (start 41.783 43.44) (end 41.783 44.356) (width 1) (layer "F.Cu") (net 11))
 (segment (start 42 64.235) (end 45.61 67.845) (width 1) (layer "F.Cu") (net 11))
 (segment (start 44.104 42.865) (end 44.104 44.225) (width 1) (layer "F.Cu") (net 11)))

